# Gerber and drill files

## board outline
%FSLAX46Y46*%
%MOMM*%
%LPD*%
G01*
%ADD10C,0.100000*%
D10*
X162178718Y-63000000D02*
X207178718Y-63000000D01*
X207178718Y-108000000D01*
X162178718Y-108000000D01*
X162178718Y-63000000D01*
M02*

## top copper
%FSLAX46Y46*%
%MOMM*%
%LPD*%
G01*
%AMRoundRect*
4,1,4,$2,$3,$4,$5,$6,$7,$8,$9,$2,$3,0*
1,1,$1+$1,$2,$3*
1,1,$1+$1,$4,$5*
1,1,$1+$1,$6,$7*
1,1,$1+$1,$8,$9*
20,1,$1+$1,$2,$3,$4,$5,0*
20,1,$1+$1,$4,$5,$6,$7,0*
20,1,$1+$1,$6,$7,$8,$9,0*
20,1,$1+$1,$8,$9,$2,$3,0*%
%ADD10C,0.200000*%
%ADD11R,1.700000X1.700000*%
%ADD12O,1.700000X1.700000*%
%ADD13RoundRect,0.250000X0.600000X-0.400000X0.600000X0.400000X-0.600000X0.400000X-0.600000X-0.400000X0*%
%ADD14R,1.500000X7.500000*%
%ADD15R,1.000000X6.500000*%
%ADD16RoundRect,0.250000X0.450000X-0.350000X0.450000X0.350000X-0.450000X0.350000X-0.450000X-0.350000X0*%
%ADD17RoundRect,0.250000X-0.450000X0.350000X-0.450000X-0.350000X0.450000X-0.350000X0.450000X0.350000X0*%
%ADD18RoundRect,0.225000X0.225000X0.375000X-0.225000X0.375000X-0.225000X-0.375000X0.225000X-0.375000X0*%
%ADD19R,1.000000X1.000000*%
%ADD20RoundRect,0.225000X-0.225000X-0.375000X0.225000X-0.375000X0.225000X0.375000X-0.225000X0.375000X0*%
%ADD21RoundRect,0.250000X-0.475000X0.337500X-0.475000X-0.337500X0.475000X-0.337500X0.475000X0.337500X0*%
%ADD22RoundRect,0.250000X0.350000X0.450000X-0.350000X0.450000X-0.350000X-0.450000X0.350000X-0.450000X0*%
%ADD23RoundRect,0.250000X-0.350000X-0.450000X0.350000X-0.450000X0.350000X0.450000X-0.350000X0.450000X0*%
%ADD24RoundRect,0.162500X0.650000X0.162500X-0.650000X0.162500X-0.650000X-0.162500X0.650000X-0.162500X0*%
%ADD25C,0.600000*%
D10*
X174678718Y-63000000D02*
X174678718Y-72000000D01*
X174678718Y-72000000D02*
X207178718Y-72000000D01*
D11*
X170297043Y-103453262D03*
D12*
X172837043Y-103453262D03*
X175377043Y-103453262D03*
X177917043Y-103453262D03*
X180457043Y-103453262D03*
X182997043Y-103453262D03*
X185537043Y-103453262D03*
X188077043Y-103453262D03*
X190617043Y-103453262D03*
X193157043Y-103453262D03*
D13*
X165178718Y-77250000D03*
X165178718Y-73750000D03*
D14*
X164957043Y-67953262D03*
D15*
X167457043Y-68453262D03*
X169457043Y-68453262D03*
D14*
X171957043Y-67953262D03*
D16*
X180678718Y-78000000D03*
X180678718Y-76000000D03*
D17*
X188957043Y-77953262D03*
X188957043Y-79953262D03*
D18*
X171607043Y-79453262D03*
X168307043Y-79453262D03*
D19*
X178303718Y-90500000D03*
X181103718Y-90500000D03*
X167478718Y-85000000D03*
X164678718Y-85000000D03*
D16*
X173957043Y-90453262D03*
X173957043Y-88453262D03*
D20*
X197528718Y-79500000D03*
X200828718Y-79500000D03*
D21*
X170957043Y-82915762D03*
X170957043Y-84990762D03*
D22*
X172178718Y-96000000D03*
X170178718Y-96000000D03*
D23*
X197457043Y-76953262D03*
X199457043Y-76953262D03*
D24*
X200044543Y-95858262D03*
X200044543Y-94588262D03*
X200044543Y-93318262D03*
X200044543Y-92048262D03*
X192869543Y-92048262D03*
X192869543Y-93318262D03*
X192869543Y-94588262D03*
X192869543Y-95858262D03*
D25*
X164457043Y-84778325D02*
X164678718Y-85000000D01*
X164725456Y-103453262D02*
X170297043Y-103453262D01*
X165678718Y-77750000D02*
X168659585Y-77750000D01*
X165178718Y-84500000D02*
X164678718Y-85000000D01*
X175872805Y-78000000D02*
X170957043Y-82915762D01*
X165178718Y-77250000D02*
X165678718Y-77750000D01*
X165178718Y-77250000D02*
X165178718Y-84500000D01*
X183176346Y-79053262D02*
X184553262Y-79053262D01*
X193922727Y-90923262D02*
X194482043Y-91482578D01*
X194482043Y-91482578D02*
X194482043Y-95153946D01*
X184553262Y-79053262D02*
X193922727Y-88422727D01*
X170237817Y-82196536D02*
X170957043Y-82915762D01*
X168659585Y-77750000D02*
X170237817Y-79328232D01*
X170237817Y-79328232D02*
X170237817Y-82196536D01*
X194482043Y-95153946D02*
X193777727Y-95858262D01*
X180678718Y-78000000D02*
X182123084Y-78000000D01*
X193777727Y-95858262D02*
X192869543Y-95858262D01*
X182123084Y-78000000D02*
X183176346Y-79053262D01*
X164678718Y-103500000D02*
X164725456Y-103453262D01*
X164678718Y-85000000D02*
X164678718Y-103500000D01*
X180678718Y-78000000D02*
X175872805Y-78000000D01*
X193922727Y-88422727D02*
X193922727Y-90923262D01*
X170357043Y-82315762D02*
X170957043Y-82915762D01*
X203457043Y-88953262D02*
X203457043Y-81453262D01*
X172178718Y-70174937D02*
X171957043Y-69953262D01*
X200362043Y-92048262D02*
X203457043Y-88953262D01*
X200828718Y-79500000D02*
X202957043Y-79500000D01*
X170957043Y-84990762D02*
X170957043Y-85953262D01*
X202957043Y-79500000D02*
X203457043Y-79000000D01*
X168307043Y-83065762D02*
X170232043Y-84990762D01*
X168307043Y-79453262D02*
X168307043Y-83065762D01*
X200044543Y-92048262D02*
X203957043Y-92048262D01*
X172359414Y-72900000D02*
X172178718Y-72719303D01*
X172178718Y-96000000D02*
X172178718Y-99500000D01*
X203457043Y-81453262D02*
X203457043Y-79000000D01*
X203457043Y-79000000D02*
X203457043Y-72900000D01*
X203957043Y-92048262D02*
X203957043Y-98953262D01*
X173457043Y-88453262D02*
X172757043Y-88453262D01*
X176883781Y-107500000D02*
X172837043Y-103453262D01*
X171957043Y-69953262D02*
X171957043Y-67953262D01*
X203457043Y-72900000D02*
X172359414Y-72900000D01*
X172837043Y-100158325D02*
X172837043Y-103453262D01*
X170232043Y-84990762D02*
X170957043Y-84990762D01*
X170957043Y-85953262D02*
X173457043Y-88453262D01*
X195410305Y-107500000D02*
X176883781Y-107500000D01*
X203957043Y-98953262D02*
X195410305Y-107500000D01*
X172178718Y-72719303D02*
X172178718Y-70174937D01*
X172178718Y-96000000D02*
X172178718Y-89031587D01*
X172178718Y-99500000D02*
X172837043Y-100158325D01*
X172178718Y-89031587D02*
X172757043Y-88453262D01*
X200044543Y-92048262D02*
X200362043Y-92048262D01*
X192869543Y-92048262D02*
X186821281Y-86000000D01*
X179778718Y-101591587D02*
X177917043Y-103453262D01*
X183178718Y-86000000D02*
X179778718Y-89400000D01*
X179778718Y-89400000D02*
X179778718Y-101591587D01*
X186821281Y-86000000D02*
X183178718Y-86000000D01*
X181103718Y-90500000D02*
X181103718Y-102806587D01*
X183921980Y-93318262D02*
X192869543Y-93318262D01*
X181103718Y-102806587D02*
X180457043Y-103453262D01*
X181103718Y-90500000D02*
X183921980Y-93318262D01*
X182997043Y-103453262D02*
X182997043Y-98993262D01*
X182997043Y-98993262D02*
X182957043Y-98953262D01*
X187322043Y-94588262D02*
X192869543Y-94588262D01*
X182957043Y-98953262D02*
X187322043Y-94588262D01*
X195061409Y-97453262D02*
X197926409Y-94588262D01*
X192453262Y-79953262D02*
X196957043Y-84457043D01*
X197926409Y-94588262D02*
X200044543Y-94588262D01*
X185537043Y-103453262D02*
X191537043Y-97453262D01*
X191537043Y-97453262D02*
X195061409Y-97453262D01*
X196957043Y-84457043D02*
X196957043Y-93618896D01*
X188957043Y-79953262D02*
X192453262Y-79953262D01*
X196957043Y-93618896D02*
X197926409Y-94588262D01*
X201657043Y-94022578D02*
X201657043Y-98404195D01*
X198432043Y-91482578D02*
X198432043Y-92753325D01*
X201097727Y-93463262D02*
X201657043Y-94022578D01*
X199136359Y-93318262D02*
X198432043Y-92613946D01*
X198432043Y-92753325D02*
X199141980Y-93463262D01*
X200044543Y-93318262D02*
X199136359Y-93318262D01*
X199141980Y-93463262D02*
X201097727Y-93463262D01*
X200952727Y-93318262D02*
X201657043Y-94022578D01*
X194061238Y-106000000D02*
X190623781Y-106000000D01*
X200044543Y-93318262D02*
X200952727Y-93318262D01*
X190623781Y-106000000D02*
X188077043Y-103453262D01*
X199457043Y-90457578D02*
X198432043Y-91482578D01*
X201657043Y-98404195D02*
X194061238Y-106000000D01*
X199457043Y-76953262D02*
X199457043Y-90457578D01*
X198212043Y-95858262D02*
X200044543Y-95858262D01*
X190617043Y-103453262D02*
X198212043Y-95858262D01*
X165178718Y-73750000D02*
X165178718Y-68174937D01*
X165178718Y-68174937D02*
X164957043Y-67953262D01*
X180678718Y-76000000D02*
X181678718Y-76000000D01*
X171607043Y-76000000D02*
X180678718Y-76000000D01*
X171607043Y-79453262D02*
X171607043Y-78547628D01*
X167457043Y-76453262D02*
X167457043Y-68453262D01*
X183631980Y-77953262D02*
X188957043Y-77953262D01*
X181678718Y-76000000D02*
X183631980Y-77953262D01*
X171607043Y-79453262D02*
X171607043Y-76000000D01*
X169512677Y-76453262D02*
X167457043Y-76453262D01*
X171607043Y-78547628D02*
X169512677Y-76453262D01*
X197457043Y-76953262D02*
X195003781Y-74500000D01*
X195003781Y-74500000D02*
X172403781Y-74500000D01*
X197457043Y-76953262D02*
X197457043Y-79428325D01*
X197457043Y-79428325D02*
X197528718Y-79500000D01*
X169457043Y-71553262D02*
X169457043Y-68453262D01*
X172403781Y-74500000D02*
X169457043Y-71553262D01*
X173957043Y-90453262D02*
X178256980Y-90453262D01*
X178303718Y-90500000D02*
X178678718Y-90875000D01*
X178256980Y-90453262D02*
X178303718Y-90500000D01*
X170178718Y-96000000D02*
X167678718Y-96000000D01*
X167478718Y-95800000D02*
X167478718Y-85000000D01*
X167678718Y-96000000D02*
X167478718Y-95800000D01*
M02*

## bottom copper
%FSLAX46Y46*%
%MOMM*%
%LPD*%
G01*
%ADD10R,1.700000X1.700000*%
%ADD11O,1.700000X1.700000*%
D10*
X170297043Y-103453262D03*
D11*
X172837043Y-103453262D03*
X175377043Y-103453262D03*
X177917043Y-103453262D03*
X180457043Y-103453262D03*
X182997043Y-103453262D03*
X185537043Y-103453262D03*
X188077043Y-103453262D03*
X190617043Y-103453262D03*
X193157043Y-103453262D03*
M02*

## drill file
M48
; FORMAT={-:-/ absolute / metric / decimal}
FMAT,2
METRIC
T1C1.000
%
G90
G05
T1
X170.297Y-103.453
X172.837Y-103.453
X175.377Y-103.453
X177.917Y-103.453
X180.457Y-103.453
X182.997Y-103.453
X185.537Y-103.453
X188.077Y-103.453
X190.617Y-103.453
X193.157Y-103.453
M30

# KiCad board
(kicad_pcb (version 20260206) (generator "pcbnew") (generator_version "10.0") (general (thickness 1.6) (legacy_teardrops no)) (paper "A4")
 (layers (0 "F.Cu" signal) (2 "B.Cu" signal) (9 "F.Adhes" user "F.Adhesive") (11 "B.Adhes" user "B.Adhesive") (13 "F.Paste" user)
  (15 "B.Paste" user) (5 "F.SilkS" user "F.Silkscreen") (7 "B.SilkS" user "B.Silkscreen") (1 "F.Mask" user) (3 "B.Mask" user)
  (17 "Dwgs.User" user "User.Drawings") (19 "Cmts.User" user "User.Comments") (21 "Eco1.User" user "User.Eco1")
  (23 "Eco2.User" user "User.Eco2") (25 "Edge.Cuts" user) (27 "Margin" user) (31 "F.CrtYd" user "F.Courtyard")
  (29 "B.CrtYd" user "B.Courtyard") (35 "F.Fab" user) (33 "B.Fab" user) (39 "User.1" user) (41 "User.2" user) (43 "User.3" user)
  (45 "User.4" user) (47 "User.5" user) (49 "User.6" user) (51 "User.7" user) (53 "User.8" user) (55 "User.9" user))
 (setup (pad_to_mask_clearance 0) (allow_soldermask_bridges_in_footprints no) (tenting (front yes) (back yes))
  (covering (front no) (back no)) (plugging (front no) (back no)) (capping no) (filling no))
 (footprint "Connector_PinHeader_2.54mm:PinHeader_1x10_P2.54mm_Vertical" (layer "F.Cu") (at 170.297043 103.453262 90)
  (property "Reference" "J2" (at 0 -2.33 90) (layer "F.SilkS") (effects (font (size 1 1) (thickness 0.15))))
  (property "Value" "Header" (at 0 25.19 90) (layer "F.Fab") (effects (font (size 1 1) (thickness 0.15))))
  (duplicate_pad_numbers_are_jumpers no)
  (pad "1" thru_hole rect (at 0 0 90) (size 1.7 1.7) (drill 1) (layers "*.Cu" "*.Mask") (remove_unused_layers no) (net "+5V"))
  (pad "2" thru_hole oval (at 0 2.54 90) (size 1.7 1.7) (drill 1) (layers "*.Cu" "*.Mask") (remove_unused_layers no) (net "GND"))
  (pad "3" thru_hole oval (at 0 5.08 90) (size 1.7 1.7) (drill 1) (layers "*.Cu" "*.Mask") (remove_unused_layers no)
   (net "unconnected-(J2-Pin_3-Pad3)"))
  (pad "4" thru_hole oval (at 0 7.62 90) (size 1.7 1.7) (drill 1) (layers "*.Cu" "*.Mask") (remove_unused_layers no) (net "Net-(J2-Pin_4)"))
  (pad "5" thru_hole oval (at 0 10.16 90) (size 1.7 1.7) (drill 1) (layers "*.Cu" "*.Mask") (remove_unused_layers no) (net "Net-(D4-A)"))
  (pad "6" thru_hole oval (at 0 12.7 90) (size 1.7 1.7) (drill 1) (layers "*.Cu" "*.Mask") (remove_unused_layers no) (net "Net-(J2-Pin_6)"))
  (pad "7" thru_hole oval (at 0 15.24 90) (size 1.7 1.7) (drill 1) (layers "*.Cu" "*.Mask") (remove_unused_layers no) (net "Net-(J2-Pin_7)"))
  (pad "8" thru_hole oval (at 0 17.78 90) (size 1.7 1.7) (drill 1) (layers "*.Cu" "*.Mask") (remove_unused_layers no) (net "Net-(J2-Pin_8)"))
  (pad "9" thru_hole oval (at 0 20.32 90) (size 1.7 1.7) (drill 1) (layers "*.Cu" "*.Mask") (remove_unused_layers no) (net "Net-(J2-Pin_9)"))
  (pad "10" thru_hole oval (at 0 22.86 90) (size 1.7 1.7) (drill 1) (layers "*.Cu" "*.Mask") (remove_unused_layers no)
   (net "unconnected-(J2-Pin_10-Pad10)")))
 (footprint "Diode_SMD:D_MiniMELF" (layer "F.Cu") (at 165.178718 75.5 90)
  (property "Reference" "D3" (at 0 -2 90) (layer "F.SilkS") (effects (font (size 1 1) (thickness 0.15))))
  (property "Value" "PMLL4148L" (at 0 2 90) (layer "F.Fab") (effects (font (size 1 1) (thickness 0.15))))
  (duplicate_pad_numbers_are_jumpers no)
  (pad "1" smd roundrect (at -1.75 0 90) (size 1.3 1.7) (layers "F.Cu" "F.Mask" "F.Paste") (roundrect_rratio 0.1923076923) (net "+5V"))
  (pad "2" smd roundrect (at 1.75 0 90) (size 1.3 1.7) (layers "F.Cu" "F.Mask" "F.Paste") (roundrect_rratio 0.1923076923) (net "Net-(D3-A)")))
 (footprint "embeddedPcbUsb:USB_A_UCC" (layer "F.Cu") (at 168.457043 68.153262 -90)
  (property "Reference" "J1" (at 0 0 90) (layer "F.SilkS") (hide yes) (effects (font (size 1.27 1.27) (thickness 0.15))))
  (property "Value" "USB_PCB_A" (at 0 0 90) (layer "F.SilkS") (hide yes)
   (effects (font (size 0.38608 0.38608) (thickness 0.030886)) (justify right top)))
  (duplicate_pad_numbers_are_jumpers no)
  (pad "1" smd rect (at -0.2 3.5 270) (size 7.5 1.5) (layers "F.Cu" "F.Mask" "F.Paste") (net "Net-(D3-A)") (solder_mask_margin 0.1016))
  (pad "2" smd rect (at 0.3 1 270) (size 6.5 1) (layers "F.Cu" "F.Mask" "F.Paste") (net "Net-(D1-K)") (solder_mask_margin 0.1016))
  (pad "3" smd rect (at 0.3 -1 270) (size 6.5 1) (layers "F.Cu" "F.Mask" "F.Paste") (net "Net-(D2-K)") (solder_mask_margin 0.1016))
  (pad "4" smd rect (at -0.2 -3.5 270) (size 7.5 1.5) (layers "F.Cu" "F.Mask" "F.Paste") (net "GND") (solder_mask_margin 0.1016)))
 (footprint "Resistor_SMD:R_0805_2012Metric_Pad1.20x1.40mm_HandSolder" (layer "F.Cu") (at 180.678718 77 90)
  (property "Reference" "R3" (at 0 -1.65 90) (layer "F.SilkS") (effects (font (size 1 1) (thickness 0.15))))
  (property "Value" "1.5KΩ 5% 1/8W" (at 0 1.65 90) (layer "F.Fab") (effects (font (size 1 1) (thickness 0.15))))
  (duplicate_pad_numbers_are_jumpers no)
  (pad "1" smd roundrect (at -1 0 90) (size 1.2 1.4) (layers "F.Cu" "F.Mask" "F.Paste") (roundrect_rratio 0.208333) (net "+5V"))
  (pad "2" smd roundrect (at 1 0 90) (size 1.2 1.4) (layers "F.Cu" "F.Mask" "F.Paste") (roundrect_rratio 0.208333) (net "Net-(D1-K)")))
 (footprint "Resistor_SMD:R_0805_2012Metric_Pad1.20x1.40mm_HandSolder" (layer "F.Cu") (at 188.957043 78.953262 -90)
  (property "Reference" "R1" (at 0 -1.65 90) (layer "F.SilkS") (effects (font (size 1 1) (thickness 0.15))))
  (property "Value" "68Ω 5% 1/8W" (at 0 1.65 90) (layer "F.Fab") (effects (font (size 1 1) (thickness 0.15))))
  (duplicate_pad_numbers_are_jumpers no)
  (pad "1" smd roundrect (at -1 0 270) (size 1.2 1.4) (layers "F.Cu" "F.Mask" "F.Paste") (roundrect_rratio 0.208333) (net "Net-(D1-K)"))
  (pad "2" smd roundrect (at 1 0 270) (size 1.2 1.4) (layers "F.Cu" "F.Mask" "F.Paste") (roundrect_rratio 0.208333) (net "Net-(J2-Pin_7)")))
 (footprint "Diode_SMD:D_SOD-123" (layer "F.Cu") (at 169.957043 79.453262 180)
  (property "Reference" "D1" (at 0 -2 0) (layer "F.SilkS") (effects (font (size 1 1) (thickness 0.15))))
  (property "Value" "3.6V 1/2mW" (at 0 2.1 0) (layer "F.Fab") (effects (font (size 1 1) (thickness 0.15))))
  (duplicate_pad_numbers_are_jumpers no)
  (pad "1" smd roundrect (at -1.65 0 180) (size 0.9 1.2) (layers "F.Cu" "F.Mask" "F.Paste") (roundrect_rratio 0.25) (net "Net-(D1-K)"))
  (pad "2" smd roundrect (at 1.65 0 180) (size 0.9 1.2) (layers "F.Cu" "F.Mask" "F.Paste") (roundrect_rratio 0.25) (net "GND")))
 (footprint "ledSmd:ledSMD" (layer "F.Cu") (at 180.103718 90.5)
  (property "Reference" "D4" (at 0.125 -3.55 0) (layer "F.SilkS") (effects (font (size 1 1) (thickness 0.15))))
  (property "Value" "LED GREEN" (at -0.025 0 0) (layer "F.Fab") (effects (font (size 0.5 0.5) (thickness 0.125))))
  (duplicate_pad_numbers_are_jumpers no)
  (pad "1" smd rect (at -1.8 0) (size 1 1) (layers "F.Cu" "F.Mask" "F.Paste") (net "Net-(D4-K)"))
  (pad "2" smd rect (at 1 0) (size 1 1) (layers "F.Cu" "F.Mask" "F.Paste") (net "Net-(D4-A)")))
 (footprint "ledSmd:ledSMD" (layer "F.Cu") (at 165.678718 85 180)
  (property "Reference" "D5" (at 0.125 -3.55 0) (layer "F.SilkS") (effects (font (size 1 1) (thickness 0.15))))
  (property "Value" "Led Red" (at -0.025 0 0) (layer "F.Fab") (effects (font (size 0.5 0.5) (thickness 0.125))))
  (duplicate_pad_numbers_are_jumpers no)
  (pad "1" smd rect (at -1.8 0 180) (size 1 1) (layers "F.Cu" "F.Mask" "F.Paste") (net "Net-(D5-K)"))
  (pad "2" smd rect (at 1 0 180) (size 1 1) (layers "F.Cu" "F.Mask" "F.Paste") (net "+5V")))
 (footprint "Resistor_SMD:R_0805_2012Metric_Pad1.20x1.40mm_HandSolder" (layer "F.Cu") (at 173.957043 89.453262 90)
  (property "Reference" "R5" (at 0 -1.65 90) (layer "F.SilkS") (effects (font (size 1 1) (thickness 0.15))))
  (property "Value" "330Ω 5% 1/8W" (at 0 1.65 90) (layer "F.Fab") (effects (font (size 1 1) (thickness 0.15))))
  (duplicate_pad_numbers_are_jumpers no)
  (pad "1" smd roundrect (at -1 0 90) (size 1.2 1.4) (layers "F.Cu" "F.Mask" "F.Paste") (roundrect_rratio 0.208333) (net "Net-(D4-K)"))
  (pad "2" smd roundrect (at 1 0 90) (size 1.2 1.4) (layers "F.Cu" "F.Mask" "F.Paste") (roundrect_rratio 0.208333) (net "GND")))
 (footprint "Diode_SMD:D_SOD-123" (layer "F.Cu") (at 199.178718 79.5)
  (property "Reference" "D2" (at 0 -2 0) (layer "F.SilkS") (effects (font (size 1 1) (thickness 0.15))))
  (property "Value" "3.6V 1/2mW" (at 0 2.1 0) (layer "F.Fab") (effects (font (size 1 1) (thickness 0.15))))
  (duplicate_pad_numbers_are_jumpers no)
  (pad "1" smd roundrect (at -1.65 0) (size 0.9 1.2) (layers "F.Cu" "F.Mask" "F.Paste") (roundrect_rratio 0.25) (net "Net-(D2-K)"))
  (pad "2" smd roundrect (at 1.65 0) (size 0.9 1.2) (layers "F.Cu" "F.Mask" "F.Paste") (roundrect_rratio 0.25) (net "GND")))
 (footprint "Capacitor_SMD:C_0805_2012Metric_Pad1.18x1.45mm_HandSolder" (layer "F.Cu") (at 170.957043 83.953262 -90)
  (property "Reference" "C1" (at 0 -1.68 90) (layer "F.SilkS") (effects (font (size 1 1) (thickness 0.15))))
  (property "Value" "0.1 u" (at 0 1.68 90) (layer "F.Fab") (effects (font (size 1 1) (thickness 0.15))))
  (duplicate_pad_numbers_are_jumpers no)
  (pad "1" smd roundrect (at -1.0375 0 270) (size 1.175 1.45) (layers "F.Cu" "F.Mask" "F.Paste") (roundrect_rratio 0.212766) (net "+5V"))
  (pad "2" smd roundrect (at 1.0375 0 270) (size 1.175 1.45) (layers "F.Cu" "F.Mask" "F.Paste") (roundrect_rratio 0.212766) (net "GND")))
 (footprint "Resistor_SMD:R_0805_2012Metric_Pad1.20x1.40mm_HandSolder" (layer "F.Cu") (at 171.178718 96 180)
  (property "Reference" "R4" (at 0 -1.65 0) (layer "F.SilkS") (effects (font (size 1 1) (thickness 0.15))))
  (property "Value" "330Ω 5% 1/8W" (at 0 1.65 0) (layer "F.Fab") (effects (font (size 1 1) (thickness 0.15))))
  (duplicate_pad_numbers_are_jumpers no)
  (pad "1" smd roundrect (at -1 0 180) (size 1.2 1.4) (layers "F.Cu" "F.Mask" "F.Paste") (roundrect_rratio 0.208333) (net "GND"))
  (pad "2" smd roundrect (at 1 0 180) (size 1.2 1.4) (layers "F.Cu" "F.Mask" "F.Paste") (roundrect_rratio 0.208333) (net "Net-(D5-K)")))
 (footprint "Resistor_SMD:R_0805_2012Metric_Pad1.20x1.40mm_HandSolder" (layer "F.Cu") (at 198.457043 76.953262)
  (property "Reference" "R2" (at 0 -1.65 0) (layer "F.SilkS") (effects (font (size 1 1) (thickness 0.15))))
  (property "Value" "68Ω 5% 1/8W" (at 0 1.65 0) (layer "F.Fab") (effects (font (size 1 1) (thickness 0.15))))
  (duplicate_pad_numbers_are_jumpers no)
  (pad "1" smd roundrect (at -1 0) (size 1.2 1.4) (layers "F.Cu" "F.Mask" "F.Paste") (roundrect_rratio 0.208333) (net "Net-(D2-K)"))
  (pad "2" smd roundrect (at 1 0) (size 1.2 1.4) (layers "F.Cu" "F.Mask" "F.Paste") (roundrect_rratio 0.208333) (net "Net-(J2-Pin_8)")))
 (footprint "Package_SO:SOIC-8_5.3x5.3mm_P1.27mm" (layer "F.Cu") (at 196.457043 93.953262 180)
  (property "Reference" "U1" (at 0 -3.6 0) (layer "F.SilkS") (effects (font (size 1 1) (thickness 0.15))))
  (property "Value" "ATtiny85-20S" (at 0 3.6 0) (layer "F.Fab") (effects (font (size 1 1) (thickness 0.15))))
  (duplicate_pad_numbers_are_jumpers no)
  (pad "1" smd roundrect (at -3.5875 -1.905 180) (size 1.625 0.65) (layers "F.Cu" "F.Mask" "F.Paste") (roundrect_rratio 0.25)
   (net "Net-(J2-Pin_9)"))
  (pad "2" smd roundrect (at -3.5875 -0.635 180) (size 1.625 0.65) (layers "F.Cu" "F.Mask" "F.Paste") (roundrect_rratio 0.25)
   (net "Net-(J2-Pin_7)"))
  (pad "3" smd roundrect (at -3.5875 0.635 180) (size 1.625 0.65) (layers "F.Cu" "F.Mask" "F.Paste") (roundrect_rratio 0.25)
   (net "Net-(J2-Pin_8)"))
  (pad "4" smd roundrect (at -3.5875 1.905 180) (size 1.625 0.65) (layers "F.Cu" "F.Mask" "F.Paste") (roundrect_rratio 0.25) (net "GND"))
  (pad "5" smd roundrect (at 3.5875 1.905 180) (size 1.625 0.65) (layers "F.Cu" "F.Mask" "F.Paste") (roundrect_rratio 0.25)
   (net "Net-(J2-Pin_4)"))
  (pad "6" smd roundrect (at 3.5875 0.635 180) (size 1.625 0.65) (layers "F.Cu" "F.Mask" "F.Paste") (roundrect_rratio 0.25)
   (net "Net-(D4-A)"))
  (pad "7" smd roundrect (at 3.5875 -0.635 180) (size 1.625 0.65) (layers "F.Cu" "F.Mask" "F.Paste") (roundrect_rratio 0.25)
   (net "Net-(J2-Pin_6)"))
  (pad "8" smd roundrect (at 3.5875 -1.905 180) (size 1.625 0.65) (layers "F.Cu" "F.Mask" "F.Paste") (roundrect_rratio 0.25) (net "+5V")))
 (gr_line (start 174.678718 63) (end 174.678718 72) (stroke (width 0.2) (type default)) (layer "F.Cu"))
 (gr_line (start 174.678718 72) (end 207.178718 72) (stroke (width 0.2) (type default)) (layer "F.Cu"))
 (gr_rect (start 162.178718 63) (end 207.178718 108) (stroke (width 0.1) (type solid)) (fill no) (layer "Edge.Cuts"))
 (segment (start 164.457043 84.778325) (end 164.678718 85) (width 0.6) (layer "F.Cu") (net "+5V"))
 (segment (start 164.725456 103.453262) (end 170.297043 103.453262) (width 0.6) (layer "F.Cu") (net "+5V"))
 (segment (start 165.678718 77.75) (end 168.659585 77.75) (width 0.6) (layer "F.Cu") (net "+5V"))
 (segment (start 165.178718 84.5) (end 164.678718 85) (width 0.6) (layer "F.Cu") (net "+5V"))
 (segment (start 175.872805 78) (end 170.957043 82.915762) (width 0.6) (layer "F.Cu") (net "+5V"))
 (segment (start 165.178718 77.25) (end 165.678718 77.75) (width 0.6) (layer "F.Cu") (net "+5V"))
 (segment (start 165.178718 77.25) (end 165.178718 84.5) (width 0.6) (layer "F.Cu") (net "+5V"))
 (segment (start 183.176346 79.053262) (end 184.553262 79.053262) (width 0.6) (layer "F.Cu") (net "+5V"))
 (segment (start 193.922727 90.923262) (end 194.482043 91.482578) (width 0.6) (layer "F.Cu") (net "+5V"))
 (segment (start 194.482043 91.482578) (end 194.482043 95.153946) (width 0.6) (layer "F.Cu") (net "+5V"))
 (segment (start 184.553262 79.053262) (end 193.922727 88.422727) (width 0.6) (layer "F.Cu") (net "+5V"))
 (segment (start 170.237817 82.196536) (end 170.957043 82.915762) (width 0.6) (layer "F.Cu") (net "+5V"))
 (segment (start 168.659585 77.75) (end 170.237817 79.328232) (width 0.6) (layer "F.Cu") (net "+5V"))
 (segment (start 170.237817 79.328232) (end 170.237817 82.196536) (width 0.6) (layer "F.Cu") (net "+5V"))
 (segment (start 194.482043 95.153946) (end 193.777727 95.858262) (width 0.6) (layer "F.Cu") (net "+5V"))
 (segment (start 180.678718 78) (end 182.123084 78) (width 0.6) (layer "F.Cu") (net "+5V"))
 (segment (start 193.777727 95.858262) (end 192.869543 95.858262) (width 0.6) (layer "F.Cu") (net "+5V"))
 (segment (start 182.123084 78) (end 183.176346 79.053262) (width 0.6) (layer "F.Cu") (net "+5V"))
 (segment (start 164.678718 103.5) (end 164.725456 103.453262) (width 0.6) (layer "F.Cu") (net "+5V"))
 (segment (start 164.678718 85) (end 164.678718 103.5) (width 0.6) (layer "F.Cu") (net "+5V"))
 (segment (start 180.678718 78) (end 175.872805 78) (width 0.6) (layer "F.Cu") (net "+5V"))
 (segment (start 193.922727 88.422727) (end 193.922727 90.923262) (width 0.6) (layer "F.Cu") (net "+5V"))
 (segment (start 170.357043 82.315762) (end 170.957043 82.915762) (width 0.6) (layer "F.Cu") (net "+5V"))
 (segment (start 203.457043 88.953262) (end 203.457043 81.453262) (width 0.6) (layer "F.Cu") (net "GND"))
 (segment (start 172.178718 70.174937) (end 171.957043 69.953262) (width 0.6) (layer "F.Cu") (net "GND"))
 (segment (start 200.362043 92.048262) (end 203.457043 88.953262) (width 0.6) (layer "F.Cu") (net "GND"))
 (segment (start 200.828718 79.5) (end 202.957043 79.5) (width 0.6) (layer "F.Cu") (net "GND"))
 (segment (start 170.957043 84.990762) (end 170.957043 85.953262) (width 0.6) (layer "F.Cu") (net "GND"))
 (segment (start 202.957043 79.5) (end 203.457043 79) (width 0.6) (layer "F.Cu") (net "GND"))
 (segment (start 168.307043 83.065762) (end 170.232043 84.990762) (width 0.6) (layer "F.Cu") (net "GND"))
 (segment (start 168.307043 79.453262) (end 168.307043 83.065762) (width 0.6) (layer "F.Cu") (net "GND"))
 (segment (start 200.044543 92.048262) (end 203.957043 92.048262) (width 0.6) (layer "F.Cu") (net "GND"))
 (segment (start 172.359414 72.9) (end 172.178718 72.719303) (width 0.6) (layer "F.Cu") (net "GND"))
 (segment (start 172.178718 96) (end 172.178718 99.5) (width 0.6) (layer "F.Cu") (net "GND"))
 (segment (start 203.457043 81.453262) (end 203.457043 79) (width 0.6) (layer "F.Cu") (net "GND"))
 (segment (start 203.457043 79) (end 203.457043 72.9) (width 0.6) (layer "F.Cu") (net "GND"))
 (segment (start 203.957043 92.048262) (end 203.957043 98.953262) (width 0.6) (layer "F.Cu") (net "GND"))
 (segment (start 173.457043 88.453262) (end 172.757043 88.453262) (width 0.6) (layer "F.Cu") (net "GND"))
 (segment (start 176.883781 107.5) (end 172.837043 103.453262) (width 0.6) (layer "F.Cu") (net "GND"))
 (segment (start 171.957043 69.953262) (end 171.957043 67.953262) (width 0.6) (layer "F.Cu") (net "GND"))
 (segment (start 203.457043 72.9) (end 172.359414 72.9) (width 0.6) (layer "F.Cu") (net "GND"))
 (segment (start 172.837043 100.158325) (end 172.837043 103.453262) (width 0.6) (layer "F.Cu") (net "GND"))
 (segment (start 170.232043 84.990762) (end 170.957043 84.990762) (width 0.6) (layer "F.Cu") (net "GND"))
 (segment (start 170.957043 85.953262) (end 173.457043 88.453262) (width 0.6) (layer "F.Cu") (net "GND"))
 (segment (start 195.410305 107.5) (end 176.883781 107.5) (width 0.6) (layer "F.Cu") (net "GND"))
 (segment (start 203.957043 98.953262) (end 195.410305 107.5) (width 0.6) (layer "F.Cu") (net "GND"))
 (segment (start 172.178718 72.719303) (end 172.178718 70.174937) (width 0.6) (layer "F.Cu") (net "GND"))
 (segment (start 172.178718 96) (end 172.178718 89.031587) (width 0.6) (layer "F.Cu") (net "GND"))
 (segment (start 172.178718 99.5) (end 172.837043 100.158325) (width 0.6) (layer "F.Cu") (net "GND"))
 (segment (start 172.178718 89.031587) (end 172.757043 88.453262) (width 0.6) (layer "F.Cu") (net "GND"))
 (segment (start 200.044543 92.048262) (end 200.362043 92.048262) (width 0.6) (layer "F.Cu") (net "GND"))
 (segment (start 192.869543 92.048262) (end 186.821281 86) (width 0.6) (layer "F.Cu") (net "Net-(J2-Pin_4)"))
 (segment (start 179.778718 101.591587) (end 177.917043 103.453262) (width 0.6) (layer "F.Cu") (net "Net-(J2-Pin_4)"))
 (segment (start 183.178718 86) (end 179.778718 89.4) (width 0.6) (layer "F.Cu") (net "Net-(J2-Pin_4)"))
 (segment (start 179.778718 89.4) (end 179.778718 101.591587) (width 0.6) (layer "F.Cu") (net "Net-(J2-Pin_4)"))
 (segment (start 186.821281 86) (end 183.178718 86) (width 0.6) (layer "F.Cu") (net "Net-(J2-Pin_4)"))
 (segment (start 181.103718 90.5) (end 181.103718 102.806587) (width 0.6) (layer "F.Cu") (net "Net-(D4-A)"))
 (segment (start 183.92198 93.318262) (end 192.869543 93.318262) (width 0.6) (layer "F.Cu") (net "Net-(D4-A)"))
 (segment (start 181.103718 102.806587) (end 180.457043 103.453262) (width 0.6) (layer "F.Cu") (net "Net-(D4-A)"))
 (segment (start 181.103718 90.5) (end 183.92198 93.318262) (width 0.6) (layer "F.Cu") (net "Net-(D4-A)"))
 (segment (start 182.997043 103.453262) (end 182.997043 98.993262) (width 0.6) (layer "F.Cu") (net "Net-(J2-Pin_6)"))
 (segment (start 182.997043 98.993262) (end 182.957043 98.953262) (width 0.6) (layer "F.Cu") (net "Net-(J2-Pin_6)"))
 (segment (start 187.322043 94.588262) (end 192.869543 94.588262) (width 0.6) (layer "F.Cu") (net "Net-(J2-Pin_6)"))
 (segment (start 182.957043 98.953262) (end 187.322043 94.588262) (width 0.6) (layer "F.Cu") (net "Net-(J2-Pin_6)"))
 (segment (start 195.061409 97.453262) (end 197.926409 94.588262) (width 0.6) (layer "F.Cu") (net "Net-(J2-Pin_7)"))
 (segment (start 192.453262 79.953262) (end 196.957043 84.457043) (width 0.6) (layer "F.Cu") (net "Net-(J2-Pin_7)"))
 (segment (start 197.926409 94.588262) (end 200.044543 94.588262) (width 0.6) (layer "F.Cu") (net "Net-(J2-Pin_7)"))
 (segment (start 185.537043 103.453262) (end 191.537043 97.453262) (width 0.6) (layer "F.Cu") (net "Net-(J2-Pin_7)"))
 (segment (start 191.537043 97.453262) (end 195.061409 97.453262) (width 0.6) (layer "F.Cu") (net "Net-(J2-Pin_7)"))
 (segment (start 196.957043 84.457043) (end 196.957043 93.618896) (width 0.6) (layer "F.Cu") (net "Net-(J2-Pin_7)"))
 (segment (start 188.957043 79.953262) (end 192.453262 79.953262) (width 0.6) (layer "F.Cu") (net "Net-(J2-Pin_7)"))
 (segment (start 196.957043 93.618896) (end 197.926409 94.588262) (width 0.6) (layer "F.Cu") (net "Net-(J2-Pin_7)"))
 (segment (start 201.657043 94.022578) (end 201.657043 98.404195) (width 0.6) (layer "F.Cu") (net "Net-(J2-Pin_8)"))
 (segment (start 198.432043 91.482578) (end 198.432043 92.753325) (width 0.6) (layer "F.Cu") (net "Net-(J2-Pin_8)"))
 (segment (start 201.097727 93.463262) (end 201.657043 94.022578) (width 0.6) (layer "F.Cu") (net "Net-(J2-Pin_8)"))
 (segment (start 199.136359 93.318262) (end 198.432043 92.613946) (width 0.6) (layer "F.Cu") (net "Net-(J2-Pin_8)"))
 (segment (start 198.432043 92.753325) (end 199.14198 93.463262) (width 0.6) (layer "F.Cu") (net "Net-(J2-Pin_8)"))
 (segment (start 200.044543 93.318262) (end 199.136359 93.318262) (width 0.6) (layer "F.Cu") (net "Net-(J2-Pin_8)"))
 (segment (start 199.14198 93.463262) (end 201.097727 93.463262) (width 0.6) (layer "F.Cu") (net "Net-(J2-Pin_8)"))
 (segment (start 200.952727 93.318262) (end 201.657043 94.022578) (width 0.6) (layer "F.Cu") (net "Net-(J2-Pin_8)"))
 (segment (start 194.061238 106) (end 190.623781 106) (width 0.6) (layer "F.Cu") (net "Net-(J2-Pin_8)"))
 (segment (start 200.044543 93.318262) (end 200.952727 93.318262) (width 0.6) (layer "F.Cu") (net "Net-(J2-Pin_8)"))
 (segment (start 190.623781 106) (end 188.077043 103.453262) (width 0.6) (layer "F.Cu") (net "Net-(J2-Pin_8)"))
 (segment (start 199.457043 90.457578) (end 198.432043 91.482578) (width 0.6) (layer "F.Cu") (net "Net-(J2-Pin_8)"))
 (segment (start 201.657043 98.404195) (end 194.061238 106) (width 0.6) (layer "F.Cu") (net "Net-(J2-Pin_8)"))
 (segment (start 199.457043 76.953262) (end 199.457043 90.457578) (width 0.6) (layer "F.Cu") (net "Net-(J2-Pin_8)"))
 (segment (start 198.212043 95.858262) (end 200.044543 95.858262) (width 0.6) (layer "F.Cu") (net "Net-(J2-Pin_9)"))
 (segment (start 190.617043 103.453262) (end 198.212043 95.858262) (width 0.6) (layer "F.Cu") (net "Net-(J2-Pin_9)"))
 (segment (start 165.178718 73.75) (end 165.178718 68.174937) (width 0.6) (layer "F.Cu") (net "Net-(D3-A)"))
 (segment (start 165.178718 68.174937) (end 164.957043 67.953262) (width 0.6) (layer "F.Cu") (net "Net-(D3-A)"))
 (segment (start 180.678718 76) (end 181.678718 76) (width 0.6) (layer "F.Cu") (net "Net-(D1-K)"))
 (segment (start 171.607043 76) (end 180.678718 76) (width 0.6) (layer "F.Cu") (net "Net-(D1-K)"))
 (segment (start 171.607043 79.453262) (end 171.607043 78.547628) (width 0.6) (layer "F.Cu") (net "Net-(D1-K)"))
 (segment (start 167.457043 76.453262) (end 167.457043 68.453262) (width 0.6) (layer "F.Cu") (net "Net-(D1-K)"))
 (segment (start 183.63198 77.953262) (end 188.957043 77.953262) (width 0.6) (layer "F.Cu") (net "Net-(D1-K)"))
 (segment (start 181.678718 76) (end 183.63198 77.953262) (width 0.6) (layer "F.Cu") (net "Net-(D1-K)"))
 (segment (start 171.607043 79.453262) (end 171.607043 76) (width 0.6) (layer "F.Cu") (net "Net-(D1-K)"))
 (segment (start 169.512677 76.453262) (end 167.457043 76.453262) (width 0.6) (layer "F.Cu") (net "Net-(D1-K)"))
 (segment (start 171.607043 78.547628) (end 169.512677 76.453262) (width 0.6) (layer "F.Cu") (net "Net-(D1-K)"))
 (segment (start 197.457043 76.953262) (end 195.003781 74.5) (width 0.6) (layer "F.Cu") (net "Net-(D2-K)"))
 (segment (start 195.003781 74.5) (end 172.403781 74.5) (width 0.6) (layer "F.Cu") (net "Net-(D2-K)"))
 (segment (start 197.457043 76.953262) (end 197.457043 79.428325) (width 0.6) (layer "F.Cu") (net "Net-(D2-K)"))
 (segment (start 197.457043 79.428325) (end 197.528718 79.5) (width 0.6) (layer "F.Cu") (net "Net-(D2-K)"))
 (segment (start 169.457043 71.553262) (end 169.457043 68.453262) (width 0.6) (layer "F.Cu") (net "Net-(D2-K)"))
 (segment (start 172.403781 74.5) (end 169.457043 71.553262) (width 0.6) (layer "F.Cu") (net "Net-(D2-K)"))
 (segment (start 173.957043 90.453262) (end 178.25698 90.453262) (width 0.6) (layer "F.Cu") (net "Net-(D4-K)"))
 (segment (start 178.303718 90.5) (end 178.678718 90.875) (width 0.6) (layer "F.Cu") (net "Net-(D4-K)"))
 (segment (start 178.25698 90.453262) (end 178.303718 90.5) (width 0.6) (layer "F.Cu") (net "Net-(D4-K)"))
 (segment (start 170.178718 96) (end 167.678718 96) (width 0.6) (layer "F.Cu") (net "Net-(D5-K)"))
 (segment (start 167.478718 95.8) (end 167.478718 85) (width 0.6) (layer "F.Cu") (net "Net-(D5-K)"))
 (segment (start 167.678718 96) (end 167.478718 95.8) (width 0.6) (layer "F.Cu") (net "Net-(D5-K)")))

